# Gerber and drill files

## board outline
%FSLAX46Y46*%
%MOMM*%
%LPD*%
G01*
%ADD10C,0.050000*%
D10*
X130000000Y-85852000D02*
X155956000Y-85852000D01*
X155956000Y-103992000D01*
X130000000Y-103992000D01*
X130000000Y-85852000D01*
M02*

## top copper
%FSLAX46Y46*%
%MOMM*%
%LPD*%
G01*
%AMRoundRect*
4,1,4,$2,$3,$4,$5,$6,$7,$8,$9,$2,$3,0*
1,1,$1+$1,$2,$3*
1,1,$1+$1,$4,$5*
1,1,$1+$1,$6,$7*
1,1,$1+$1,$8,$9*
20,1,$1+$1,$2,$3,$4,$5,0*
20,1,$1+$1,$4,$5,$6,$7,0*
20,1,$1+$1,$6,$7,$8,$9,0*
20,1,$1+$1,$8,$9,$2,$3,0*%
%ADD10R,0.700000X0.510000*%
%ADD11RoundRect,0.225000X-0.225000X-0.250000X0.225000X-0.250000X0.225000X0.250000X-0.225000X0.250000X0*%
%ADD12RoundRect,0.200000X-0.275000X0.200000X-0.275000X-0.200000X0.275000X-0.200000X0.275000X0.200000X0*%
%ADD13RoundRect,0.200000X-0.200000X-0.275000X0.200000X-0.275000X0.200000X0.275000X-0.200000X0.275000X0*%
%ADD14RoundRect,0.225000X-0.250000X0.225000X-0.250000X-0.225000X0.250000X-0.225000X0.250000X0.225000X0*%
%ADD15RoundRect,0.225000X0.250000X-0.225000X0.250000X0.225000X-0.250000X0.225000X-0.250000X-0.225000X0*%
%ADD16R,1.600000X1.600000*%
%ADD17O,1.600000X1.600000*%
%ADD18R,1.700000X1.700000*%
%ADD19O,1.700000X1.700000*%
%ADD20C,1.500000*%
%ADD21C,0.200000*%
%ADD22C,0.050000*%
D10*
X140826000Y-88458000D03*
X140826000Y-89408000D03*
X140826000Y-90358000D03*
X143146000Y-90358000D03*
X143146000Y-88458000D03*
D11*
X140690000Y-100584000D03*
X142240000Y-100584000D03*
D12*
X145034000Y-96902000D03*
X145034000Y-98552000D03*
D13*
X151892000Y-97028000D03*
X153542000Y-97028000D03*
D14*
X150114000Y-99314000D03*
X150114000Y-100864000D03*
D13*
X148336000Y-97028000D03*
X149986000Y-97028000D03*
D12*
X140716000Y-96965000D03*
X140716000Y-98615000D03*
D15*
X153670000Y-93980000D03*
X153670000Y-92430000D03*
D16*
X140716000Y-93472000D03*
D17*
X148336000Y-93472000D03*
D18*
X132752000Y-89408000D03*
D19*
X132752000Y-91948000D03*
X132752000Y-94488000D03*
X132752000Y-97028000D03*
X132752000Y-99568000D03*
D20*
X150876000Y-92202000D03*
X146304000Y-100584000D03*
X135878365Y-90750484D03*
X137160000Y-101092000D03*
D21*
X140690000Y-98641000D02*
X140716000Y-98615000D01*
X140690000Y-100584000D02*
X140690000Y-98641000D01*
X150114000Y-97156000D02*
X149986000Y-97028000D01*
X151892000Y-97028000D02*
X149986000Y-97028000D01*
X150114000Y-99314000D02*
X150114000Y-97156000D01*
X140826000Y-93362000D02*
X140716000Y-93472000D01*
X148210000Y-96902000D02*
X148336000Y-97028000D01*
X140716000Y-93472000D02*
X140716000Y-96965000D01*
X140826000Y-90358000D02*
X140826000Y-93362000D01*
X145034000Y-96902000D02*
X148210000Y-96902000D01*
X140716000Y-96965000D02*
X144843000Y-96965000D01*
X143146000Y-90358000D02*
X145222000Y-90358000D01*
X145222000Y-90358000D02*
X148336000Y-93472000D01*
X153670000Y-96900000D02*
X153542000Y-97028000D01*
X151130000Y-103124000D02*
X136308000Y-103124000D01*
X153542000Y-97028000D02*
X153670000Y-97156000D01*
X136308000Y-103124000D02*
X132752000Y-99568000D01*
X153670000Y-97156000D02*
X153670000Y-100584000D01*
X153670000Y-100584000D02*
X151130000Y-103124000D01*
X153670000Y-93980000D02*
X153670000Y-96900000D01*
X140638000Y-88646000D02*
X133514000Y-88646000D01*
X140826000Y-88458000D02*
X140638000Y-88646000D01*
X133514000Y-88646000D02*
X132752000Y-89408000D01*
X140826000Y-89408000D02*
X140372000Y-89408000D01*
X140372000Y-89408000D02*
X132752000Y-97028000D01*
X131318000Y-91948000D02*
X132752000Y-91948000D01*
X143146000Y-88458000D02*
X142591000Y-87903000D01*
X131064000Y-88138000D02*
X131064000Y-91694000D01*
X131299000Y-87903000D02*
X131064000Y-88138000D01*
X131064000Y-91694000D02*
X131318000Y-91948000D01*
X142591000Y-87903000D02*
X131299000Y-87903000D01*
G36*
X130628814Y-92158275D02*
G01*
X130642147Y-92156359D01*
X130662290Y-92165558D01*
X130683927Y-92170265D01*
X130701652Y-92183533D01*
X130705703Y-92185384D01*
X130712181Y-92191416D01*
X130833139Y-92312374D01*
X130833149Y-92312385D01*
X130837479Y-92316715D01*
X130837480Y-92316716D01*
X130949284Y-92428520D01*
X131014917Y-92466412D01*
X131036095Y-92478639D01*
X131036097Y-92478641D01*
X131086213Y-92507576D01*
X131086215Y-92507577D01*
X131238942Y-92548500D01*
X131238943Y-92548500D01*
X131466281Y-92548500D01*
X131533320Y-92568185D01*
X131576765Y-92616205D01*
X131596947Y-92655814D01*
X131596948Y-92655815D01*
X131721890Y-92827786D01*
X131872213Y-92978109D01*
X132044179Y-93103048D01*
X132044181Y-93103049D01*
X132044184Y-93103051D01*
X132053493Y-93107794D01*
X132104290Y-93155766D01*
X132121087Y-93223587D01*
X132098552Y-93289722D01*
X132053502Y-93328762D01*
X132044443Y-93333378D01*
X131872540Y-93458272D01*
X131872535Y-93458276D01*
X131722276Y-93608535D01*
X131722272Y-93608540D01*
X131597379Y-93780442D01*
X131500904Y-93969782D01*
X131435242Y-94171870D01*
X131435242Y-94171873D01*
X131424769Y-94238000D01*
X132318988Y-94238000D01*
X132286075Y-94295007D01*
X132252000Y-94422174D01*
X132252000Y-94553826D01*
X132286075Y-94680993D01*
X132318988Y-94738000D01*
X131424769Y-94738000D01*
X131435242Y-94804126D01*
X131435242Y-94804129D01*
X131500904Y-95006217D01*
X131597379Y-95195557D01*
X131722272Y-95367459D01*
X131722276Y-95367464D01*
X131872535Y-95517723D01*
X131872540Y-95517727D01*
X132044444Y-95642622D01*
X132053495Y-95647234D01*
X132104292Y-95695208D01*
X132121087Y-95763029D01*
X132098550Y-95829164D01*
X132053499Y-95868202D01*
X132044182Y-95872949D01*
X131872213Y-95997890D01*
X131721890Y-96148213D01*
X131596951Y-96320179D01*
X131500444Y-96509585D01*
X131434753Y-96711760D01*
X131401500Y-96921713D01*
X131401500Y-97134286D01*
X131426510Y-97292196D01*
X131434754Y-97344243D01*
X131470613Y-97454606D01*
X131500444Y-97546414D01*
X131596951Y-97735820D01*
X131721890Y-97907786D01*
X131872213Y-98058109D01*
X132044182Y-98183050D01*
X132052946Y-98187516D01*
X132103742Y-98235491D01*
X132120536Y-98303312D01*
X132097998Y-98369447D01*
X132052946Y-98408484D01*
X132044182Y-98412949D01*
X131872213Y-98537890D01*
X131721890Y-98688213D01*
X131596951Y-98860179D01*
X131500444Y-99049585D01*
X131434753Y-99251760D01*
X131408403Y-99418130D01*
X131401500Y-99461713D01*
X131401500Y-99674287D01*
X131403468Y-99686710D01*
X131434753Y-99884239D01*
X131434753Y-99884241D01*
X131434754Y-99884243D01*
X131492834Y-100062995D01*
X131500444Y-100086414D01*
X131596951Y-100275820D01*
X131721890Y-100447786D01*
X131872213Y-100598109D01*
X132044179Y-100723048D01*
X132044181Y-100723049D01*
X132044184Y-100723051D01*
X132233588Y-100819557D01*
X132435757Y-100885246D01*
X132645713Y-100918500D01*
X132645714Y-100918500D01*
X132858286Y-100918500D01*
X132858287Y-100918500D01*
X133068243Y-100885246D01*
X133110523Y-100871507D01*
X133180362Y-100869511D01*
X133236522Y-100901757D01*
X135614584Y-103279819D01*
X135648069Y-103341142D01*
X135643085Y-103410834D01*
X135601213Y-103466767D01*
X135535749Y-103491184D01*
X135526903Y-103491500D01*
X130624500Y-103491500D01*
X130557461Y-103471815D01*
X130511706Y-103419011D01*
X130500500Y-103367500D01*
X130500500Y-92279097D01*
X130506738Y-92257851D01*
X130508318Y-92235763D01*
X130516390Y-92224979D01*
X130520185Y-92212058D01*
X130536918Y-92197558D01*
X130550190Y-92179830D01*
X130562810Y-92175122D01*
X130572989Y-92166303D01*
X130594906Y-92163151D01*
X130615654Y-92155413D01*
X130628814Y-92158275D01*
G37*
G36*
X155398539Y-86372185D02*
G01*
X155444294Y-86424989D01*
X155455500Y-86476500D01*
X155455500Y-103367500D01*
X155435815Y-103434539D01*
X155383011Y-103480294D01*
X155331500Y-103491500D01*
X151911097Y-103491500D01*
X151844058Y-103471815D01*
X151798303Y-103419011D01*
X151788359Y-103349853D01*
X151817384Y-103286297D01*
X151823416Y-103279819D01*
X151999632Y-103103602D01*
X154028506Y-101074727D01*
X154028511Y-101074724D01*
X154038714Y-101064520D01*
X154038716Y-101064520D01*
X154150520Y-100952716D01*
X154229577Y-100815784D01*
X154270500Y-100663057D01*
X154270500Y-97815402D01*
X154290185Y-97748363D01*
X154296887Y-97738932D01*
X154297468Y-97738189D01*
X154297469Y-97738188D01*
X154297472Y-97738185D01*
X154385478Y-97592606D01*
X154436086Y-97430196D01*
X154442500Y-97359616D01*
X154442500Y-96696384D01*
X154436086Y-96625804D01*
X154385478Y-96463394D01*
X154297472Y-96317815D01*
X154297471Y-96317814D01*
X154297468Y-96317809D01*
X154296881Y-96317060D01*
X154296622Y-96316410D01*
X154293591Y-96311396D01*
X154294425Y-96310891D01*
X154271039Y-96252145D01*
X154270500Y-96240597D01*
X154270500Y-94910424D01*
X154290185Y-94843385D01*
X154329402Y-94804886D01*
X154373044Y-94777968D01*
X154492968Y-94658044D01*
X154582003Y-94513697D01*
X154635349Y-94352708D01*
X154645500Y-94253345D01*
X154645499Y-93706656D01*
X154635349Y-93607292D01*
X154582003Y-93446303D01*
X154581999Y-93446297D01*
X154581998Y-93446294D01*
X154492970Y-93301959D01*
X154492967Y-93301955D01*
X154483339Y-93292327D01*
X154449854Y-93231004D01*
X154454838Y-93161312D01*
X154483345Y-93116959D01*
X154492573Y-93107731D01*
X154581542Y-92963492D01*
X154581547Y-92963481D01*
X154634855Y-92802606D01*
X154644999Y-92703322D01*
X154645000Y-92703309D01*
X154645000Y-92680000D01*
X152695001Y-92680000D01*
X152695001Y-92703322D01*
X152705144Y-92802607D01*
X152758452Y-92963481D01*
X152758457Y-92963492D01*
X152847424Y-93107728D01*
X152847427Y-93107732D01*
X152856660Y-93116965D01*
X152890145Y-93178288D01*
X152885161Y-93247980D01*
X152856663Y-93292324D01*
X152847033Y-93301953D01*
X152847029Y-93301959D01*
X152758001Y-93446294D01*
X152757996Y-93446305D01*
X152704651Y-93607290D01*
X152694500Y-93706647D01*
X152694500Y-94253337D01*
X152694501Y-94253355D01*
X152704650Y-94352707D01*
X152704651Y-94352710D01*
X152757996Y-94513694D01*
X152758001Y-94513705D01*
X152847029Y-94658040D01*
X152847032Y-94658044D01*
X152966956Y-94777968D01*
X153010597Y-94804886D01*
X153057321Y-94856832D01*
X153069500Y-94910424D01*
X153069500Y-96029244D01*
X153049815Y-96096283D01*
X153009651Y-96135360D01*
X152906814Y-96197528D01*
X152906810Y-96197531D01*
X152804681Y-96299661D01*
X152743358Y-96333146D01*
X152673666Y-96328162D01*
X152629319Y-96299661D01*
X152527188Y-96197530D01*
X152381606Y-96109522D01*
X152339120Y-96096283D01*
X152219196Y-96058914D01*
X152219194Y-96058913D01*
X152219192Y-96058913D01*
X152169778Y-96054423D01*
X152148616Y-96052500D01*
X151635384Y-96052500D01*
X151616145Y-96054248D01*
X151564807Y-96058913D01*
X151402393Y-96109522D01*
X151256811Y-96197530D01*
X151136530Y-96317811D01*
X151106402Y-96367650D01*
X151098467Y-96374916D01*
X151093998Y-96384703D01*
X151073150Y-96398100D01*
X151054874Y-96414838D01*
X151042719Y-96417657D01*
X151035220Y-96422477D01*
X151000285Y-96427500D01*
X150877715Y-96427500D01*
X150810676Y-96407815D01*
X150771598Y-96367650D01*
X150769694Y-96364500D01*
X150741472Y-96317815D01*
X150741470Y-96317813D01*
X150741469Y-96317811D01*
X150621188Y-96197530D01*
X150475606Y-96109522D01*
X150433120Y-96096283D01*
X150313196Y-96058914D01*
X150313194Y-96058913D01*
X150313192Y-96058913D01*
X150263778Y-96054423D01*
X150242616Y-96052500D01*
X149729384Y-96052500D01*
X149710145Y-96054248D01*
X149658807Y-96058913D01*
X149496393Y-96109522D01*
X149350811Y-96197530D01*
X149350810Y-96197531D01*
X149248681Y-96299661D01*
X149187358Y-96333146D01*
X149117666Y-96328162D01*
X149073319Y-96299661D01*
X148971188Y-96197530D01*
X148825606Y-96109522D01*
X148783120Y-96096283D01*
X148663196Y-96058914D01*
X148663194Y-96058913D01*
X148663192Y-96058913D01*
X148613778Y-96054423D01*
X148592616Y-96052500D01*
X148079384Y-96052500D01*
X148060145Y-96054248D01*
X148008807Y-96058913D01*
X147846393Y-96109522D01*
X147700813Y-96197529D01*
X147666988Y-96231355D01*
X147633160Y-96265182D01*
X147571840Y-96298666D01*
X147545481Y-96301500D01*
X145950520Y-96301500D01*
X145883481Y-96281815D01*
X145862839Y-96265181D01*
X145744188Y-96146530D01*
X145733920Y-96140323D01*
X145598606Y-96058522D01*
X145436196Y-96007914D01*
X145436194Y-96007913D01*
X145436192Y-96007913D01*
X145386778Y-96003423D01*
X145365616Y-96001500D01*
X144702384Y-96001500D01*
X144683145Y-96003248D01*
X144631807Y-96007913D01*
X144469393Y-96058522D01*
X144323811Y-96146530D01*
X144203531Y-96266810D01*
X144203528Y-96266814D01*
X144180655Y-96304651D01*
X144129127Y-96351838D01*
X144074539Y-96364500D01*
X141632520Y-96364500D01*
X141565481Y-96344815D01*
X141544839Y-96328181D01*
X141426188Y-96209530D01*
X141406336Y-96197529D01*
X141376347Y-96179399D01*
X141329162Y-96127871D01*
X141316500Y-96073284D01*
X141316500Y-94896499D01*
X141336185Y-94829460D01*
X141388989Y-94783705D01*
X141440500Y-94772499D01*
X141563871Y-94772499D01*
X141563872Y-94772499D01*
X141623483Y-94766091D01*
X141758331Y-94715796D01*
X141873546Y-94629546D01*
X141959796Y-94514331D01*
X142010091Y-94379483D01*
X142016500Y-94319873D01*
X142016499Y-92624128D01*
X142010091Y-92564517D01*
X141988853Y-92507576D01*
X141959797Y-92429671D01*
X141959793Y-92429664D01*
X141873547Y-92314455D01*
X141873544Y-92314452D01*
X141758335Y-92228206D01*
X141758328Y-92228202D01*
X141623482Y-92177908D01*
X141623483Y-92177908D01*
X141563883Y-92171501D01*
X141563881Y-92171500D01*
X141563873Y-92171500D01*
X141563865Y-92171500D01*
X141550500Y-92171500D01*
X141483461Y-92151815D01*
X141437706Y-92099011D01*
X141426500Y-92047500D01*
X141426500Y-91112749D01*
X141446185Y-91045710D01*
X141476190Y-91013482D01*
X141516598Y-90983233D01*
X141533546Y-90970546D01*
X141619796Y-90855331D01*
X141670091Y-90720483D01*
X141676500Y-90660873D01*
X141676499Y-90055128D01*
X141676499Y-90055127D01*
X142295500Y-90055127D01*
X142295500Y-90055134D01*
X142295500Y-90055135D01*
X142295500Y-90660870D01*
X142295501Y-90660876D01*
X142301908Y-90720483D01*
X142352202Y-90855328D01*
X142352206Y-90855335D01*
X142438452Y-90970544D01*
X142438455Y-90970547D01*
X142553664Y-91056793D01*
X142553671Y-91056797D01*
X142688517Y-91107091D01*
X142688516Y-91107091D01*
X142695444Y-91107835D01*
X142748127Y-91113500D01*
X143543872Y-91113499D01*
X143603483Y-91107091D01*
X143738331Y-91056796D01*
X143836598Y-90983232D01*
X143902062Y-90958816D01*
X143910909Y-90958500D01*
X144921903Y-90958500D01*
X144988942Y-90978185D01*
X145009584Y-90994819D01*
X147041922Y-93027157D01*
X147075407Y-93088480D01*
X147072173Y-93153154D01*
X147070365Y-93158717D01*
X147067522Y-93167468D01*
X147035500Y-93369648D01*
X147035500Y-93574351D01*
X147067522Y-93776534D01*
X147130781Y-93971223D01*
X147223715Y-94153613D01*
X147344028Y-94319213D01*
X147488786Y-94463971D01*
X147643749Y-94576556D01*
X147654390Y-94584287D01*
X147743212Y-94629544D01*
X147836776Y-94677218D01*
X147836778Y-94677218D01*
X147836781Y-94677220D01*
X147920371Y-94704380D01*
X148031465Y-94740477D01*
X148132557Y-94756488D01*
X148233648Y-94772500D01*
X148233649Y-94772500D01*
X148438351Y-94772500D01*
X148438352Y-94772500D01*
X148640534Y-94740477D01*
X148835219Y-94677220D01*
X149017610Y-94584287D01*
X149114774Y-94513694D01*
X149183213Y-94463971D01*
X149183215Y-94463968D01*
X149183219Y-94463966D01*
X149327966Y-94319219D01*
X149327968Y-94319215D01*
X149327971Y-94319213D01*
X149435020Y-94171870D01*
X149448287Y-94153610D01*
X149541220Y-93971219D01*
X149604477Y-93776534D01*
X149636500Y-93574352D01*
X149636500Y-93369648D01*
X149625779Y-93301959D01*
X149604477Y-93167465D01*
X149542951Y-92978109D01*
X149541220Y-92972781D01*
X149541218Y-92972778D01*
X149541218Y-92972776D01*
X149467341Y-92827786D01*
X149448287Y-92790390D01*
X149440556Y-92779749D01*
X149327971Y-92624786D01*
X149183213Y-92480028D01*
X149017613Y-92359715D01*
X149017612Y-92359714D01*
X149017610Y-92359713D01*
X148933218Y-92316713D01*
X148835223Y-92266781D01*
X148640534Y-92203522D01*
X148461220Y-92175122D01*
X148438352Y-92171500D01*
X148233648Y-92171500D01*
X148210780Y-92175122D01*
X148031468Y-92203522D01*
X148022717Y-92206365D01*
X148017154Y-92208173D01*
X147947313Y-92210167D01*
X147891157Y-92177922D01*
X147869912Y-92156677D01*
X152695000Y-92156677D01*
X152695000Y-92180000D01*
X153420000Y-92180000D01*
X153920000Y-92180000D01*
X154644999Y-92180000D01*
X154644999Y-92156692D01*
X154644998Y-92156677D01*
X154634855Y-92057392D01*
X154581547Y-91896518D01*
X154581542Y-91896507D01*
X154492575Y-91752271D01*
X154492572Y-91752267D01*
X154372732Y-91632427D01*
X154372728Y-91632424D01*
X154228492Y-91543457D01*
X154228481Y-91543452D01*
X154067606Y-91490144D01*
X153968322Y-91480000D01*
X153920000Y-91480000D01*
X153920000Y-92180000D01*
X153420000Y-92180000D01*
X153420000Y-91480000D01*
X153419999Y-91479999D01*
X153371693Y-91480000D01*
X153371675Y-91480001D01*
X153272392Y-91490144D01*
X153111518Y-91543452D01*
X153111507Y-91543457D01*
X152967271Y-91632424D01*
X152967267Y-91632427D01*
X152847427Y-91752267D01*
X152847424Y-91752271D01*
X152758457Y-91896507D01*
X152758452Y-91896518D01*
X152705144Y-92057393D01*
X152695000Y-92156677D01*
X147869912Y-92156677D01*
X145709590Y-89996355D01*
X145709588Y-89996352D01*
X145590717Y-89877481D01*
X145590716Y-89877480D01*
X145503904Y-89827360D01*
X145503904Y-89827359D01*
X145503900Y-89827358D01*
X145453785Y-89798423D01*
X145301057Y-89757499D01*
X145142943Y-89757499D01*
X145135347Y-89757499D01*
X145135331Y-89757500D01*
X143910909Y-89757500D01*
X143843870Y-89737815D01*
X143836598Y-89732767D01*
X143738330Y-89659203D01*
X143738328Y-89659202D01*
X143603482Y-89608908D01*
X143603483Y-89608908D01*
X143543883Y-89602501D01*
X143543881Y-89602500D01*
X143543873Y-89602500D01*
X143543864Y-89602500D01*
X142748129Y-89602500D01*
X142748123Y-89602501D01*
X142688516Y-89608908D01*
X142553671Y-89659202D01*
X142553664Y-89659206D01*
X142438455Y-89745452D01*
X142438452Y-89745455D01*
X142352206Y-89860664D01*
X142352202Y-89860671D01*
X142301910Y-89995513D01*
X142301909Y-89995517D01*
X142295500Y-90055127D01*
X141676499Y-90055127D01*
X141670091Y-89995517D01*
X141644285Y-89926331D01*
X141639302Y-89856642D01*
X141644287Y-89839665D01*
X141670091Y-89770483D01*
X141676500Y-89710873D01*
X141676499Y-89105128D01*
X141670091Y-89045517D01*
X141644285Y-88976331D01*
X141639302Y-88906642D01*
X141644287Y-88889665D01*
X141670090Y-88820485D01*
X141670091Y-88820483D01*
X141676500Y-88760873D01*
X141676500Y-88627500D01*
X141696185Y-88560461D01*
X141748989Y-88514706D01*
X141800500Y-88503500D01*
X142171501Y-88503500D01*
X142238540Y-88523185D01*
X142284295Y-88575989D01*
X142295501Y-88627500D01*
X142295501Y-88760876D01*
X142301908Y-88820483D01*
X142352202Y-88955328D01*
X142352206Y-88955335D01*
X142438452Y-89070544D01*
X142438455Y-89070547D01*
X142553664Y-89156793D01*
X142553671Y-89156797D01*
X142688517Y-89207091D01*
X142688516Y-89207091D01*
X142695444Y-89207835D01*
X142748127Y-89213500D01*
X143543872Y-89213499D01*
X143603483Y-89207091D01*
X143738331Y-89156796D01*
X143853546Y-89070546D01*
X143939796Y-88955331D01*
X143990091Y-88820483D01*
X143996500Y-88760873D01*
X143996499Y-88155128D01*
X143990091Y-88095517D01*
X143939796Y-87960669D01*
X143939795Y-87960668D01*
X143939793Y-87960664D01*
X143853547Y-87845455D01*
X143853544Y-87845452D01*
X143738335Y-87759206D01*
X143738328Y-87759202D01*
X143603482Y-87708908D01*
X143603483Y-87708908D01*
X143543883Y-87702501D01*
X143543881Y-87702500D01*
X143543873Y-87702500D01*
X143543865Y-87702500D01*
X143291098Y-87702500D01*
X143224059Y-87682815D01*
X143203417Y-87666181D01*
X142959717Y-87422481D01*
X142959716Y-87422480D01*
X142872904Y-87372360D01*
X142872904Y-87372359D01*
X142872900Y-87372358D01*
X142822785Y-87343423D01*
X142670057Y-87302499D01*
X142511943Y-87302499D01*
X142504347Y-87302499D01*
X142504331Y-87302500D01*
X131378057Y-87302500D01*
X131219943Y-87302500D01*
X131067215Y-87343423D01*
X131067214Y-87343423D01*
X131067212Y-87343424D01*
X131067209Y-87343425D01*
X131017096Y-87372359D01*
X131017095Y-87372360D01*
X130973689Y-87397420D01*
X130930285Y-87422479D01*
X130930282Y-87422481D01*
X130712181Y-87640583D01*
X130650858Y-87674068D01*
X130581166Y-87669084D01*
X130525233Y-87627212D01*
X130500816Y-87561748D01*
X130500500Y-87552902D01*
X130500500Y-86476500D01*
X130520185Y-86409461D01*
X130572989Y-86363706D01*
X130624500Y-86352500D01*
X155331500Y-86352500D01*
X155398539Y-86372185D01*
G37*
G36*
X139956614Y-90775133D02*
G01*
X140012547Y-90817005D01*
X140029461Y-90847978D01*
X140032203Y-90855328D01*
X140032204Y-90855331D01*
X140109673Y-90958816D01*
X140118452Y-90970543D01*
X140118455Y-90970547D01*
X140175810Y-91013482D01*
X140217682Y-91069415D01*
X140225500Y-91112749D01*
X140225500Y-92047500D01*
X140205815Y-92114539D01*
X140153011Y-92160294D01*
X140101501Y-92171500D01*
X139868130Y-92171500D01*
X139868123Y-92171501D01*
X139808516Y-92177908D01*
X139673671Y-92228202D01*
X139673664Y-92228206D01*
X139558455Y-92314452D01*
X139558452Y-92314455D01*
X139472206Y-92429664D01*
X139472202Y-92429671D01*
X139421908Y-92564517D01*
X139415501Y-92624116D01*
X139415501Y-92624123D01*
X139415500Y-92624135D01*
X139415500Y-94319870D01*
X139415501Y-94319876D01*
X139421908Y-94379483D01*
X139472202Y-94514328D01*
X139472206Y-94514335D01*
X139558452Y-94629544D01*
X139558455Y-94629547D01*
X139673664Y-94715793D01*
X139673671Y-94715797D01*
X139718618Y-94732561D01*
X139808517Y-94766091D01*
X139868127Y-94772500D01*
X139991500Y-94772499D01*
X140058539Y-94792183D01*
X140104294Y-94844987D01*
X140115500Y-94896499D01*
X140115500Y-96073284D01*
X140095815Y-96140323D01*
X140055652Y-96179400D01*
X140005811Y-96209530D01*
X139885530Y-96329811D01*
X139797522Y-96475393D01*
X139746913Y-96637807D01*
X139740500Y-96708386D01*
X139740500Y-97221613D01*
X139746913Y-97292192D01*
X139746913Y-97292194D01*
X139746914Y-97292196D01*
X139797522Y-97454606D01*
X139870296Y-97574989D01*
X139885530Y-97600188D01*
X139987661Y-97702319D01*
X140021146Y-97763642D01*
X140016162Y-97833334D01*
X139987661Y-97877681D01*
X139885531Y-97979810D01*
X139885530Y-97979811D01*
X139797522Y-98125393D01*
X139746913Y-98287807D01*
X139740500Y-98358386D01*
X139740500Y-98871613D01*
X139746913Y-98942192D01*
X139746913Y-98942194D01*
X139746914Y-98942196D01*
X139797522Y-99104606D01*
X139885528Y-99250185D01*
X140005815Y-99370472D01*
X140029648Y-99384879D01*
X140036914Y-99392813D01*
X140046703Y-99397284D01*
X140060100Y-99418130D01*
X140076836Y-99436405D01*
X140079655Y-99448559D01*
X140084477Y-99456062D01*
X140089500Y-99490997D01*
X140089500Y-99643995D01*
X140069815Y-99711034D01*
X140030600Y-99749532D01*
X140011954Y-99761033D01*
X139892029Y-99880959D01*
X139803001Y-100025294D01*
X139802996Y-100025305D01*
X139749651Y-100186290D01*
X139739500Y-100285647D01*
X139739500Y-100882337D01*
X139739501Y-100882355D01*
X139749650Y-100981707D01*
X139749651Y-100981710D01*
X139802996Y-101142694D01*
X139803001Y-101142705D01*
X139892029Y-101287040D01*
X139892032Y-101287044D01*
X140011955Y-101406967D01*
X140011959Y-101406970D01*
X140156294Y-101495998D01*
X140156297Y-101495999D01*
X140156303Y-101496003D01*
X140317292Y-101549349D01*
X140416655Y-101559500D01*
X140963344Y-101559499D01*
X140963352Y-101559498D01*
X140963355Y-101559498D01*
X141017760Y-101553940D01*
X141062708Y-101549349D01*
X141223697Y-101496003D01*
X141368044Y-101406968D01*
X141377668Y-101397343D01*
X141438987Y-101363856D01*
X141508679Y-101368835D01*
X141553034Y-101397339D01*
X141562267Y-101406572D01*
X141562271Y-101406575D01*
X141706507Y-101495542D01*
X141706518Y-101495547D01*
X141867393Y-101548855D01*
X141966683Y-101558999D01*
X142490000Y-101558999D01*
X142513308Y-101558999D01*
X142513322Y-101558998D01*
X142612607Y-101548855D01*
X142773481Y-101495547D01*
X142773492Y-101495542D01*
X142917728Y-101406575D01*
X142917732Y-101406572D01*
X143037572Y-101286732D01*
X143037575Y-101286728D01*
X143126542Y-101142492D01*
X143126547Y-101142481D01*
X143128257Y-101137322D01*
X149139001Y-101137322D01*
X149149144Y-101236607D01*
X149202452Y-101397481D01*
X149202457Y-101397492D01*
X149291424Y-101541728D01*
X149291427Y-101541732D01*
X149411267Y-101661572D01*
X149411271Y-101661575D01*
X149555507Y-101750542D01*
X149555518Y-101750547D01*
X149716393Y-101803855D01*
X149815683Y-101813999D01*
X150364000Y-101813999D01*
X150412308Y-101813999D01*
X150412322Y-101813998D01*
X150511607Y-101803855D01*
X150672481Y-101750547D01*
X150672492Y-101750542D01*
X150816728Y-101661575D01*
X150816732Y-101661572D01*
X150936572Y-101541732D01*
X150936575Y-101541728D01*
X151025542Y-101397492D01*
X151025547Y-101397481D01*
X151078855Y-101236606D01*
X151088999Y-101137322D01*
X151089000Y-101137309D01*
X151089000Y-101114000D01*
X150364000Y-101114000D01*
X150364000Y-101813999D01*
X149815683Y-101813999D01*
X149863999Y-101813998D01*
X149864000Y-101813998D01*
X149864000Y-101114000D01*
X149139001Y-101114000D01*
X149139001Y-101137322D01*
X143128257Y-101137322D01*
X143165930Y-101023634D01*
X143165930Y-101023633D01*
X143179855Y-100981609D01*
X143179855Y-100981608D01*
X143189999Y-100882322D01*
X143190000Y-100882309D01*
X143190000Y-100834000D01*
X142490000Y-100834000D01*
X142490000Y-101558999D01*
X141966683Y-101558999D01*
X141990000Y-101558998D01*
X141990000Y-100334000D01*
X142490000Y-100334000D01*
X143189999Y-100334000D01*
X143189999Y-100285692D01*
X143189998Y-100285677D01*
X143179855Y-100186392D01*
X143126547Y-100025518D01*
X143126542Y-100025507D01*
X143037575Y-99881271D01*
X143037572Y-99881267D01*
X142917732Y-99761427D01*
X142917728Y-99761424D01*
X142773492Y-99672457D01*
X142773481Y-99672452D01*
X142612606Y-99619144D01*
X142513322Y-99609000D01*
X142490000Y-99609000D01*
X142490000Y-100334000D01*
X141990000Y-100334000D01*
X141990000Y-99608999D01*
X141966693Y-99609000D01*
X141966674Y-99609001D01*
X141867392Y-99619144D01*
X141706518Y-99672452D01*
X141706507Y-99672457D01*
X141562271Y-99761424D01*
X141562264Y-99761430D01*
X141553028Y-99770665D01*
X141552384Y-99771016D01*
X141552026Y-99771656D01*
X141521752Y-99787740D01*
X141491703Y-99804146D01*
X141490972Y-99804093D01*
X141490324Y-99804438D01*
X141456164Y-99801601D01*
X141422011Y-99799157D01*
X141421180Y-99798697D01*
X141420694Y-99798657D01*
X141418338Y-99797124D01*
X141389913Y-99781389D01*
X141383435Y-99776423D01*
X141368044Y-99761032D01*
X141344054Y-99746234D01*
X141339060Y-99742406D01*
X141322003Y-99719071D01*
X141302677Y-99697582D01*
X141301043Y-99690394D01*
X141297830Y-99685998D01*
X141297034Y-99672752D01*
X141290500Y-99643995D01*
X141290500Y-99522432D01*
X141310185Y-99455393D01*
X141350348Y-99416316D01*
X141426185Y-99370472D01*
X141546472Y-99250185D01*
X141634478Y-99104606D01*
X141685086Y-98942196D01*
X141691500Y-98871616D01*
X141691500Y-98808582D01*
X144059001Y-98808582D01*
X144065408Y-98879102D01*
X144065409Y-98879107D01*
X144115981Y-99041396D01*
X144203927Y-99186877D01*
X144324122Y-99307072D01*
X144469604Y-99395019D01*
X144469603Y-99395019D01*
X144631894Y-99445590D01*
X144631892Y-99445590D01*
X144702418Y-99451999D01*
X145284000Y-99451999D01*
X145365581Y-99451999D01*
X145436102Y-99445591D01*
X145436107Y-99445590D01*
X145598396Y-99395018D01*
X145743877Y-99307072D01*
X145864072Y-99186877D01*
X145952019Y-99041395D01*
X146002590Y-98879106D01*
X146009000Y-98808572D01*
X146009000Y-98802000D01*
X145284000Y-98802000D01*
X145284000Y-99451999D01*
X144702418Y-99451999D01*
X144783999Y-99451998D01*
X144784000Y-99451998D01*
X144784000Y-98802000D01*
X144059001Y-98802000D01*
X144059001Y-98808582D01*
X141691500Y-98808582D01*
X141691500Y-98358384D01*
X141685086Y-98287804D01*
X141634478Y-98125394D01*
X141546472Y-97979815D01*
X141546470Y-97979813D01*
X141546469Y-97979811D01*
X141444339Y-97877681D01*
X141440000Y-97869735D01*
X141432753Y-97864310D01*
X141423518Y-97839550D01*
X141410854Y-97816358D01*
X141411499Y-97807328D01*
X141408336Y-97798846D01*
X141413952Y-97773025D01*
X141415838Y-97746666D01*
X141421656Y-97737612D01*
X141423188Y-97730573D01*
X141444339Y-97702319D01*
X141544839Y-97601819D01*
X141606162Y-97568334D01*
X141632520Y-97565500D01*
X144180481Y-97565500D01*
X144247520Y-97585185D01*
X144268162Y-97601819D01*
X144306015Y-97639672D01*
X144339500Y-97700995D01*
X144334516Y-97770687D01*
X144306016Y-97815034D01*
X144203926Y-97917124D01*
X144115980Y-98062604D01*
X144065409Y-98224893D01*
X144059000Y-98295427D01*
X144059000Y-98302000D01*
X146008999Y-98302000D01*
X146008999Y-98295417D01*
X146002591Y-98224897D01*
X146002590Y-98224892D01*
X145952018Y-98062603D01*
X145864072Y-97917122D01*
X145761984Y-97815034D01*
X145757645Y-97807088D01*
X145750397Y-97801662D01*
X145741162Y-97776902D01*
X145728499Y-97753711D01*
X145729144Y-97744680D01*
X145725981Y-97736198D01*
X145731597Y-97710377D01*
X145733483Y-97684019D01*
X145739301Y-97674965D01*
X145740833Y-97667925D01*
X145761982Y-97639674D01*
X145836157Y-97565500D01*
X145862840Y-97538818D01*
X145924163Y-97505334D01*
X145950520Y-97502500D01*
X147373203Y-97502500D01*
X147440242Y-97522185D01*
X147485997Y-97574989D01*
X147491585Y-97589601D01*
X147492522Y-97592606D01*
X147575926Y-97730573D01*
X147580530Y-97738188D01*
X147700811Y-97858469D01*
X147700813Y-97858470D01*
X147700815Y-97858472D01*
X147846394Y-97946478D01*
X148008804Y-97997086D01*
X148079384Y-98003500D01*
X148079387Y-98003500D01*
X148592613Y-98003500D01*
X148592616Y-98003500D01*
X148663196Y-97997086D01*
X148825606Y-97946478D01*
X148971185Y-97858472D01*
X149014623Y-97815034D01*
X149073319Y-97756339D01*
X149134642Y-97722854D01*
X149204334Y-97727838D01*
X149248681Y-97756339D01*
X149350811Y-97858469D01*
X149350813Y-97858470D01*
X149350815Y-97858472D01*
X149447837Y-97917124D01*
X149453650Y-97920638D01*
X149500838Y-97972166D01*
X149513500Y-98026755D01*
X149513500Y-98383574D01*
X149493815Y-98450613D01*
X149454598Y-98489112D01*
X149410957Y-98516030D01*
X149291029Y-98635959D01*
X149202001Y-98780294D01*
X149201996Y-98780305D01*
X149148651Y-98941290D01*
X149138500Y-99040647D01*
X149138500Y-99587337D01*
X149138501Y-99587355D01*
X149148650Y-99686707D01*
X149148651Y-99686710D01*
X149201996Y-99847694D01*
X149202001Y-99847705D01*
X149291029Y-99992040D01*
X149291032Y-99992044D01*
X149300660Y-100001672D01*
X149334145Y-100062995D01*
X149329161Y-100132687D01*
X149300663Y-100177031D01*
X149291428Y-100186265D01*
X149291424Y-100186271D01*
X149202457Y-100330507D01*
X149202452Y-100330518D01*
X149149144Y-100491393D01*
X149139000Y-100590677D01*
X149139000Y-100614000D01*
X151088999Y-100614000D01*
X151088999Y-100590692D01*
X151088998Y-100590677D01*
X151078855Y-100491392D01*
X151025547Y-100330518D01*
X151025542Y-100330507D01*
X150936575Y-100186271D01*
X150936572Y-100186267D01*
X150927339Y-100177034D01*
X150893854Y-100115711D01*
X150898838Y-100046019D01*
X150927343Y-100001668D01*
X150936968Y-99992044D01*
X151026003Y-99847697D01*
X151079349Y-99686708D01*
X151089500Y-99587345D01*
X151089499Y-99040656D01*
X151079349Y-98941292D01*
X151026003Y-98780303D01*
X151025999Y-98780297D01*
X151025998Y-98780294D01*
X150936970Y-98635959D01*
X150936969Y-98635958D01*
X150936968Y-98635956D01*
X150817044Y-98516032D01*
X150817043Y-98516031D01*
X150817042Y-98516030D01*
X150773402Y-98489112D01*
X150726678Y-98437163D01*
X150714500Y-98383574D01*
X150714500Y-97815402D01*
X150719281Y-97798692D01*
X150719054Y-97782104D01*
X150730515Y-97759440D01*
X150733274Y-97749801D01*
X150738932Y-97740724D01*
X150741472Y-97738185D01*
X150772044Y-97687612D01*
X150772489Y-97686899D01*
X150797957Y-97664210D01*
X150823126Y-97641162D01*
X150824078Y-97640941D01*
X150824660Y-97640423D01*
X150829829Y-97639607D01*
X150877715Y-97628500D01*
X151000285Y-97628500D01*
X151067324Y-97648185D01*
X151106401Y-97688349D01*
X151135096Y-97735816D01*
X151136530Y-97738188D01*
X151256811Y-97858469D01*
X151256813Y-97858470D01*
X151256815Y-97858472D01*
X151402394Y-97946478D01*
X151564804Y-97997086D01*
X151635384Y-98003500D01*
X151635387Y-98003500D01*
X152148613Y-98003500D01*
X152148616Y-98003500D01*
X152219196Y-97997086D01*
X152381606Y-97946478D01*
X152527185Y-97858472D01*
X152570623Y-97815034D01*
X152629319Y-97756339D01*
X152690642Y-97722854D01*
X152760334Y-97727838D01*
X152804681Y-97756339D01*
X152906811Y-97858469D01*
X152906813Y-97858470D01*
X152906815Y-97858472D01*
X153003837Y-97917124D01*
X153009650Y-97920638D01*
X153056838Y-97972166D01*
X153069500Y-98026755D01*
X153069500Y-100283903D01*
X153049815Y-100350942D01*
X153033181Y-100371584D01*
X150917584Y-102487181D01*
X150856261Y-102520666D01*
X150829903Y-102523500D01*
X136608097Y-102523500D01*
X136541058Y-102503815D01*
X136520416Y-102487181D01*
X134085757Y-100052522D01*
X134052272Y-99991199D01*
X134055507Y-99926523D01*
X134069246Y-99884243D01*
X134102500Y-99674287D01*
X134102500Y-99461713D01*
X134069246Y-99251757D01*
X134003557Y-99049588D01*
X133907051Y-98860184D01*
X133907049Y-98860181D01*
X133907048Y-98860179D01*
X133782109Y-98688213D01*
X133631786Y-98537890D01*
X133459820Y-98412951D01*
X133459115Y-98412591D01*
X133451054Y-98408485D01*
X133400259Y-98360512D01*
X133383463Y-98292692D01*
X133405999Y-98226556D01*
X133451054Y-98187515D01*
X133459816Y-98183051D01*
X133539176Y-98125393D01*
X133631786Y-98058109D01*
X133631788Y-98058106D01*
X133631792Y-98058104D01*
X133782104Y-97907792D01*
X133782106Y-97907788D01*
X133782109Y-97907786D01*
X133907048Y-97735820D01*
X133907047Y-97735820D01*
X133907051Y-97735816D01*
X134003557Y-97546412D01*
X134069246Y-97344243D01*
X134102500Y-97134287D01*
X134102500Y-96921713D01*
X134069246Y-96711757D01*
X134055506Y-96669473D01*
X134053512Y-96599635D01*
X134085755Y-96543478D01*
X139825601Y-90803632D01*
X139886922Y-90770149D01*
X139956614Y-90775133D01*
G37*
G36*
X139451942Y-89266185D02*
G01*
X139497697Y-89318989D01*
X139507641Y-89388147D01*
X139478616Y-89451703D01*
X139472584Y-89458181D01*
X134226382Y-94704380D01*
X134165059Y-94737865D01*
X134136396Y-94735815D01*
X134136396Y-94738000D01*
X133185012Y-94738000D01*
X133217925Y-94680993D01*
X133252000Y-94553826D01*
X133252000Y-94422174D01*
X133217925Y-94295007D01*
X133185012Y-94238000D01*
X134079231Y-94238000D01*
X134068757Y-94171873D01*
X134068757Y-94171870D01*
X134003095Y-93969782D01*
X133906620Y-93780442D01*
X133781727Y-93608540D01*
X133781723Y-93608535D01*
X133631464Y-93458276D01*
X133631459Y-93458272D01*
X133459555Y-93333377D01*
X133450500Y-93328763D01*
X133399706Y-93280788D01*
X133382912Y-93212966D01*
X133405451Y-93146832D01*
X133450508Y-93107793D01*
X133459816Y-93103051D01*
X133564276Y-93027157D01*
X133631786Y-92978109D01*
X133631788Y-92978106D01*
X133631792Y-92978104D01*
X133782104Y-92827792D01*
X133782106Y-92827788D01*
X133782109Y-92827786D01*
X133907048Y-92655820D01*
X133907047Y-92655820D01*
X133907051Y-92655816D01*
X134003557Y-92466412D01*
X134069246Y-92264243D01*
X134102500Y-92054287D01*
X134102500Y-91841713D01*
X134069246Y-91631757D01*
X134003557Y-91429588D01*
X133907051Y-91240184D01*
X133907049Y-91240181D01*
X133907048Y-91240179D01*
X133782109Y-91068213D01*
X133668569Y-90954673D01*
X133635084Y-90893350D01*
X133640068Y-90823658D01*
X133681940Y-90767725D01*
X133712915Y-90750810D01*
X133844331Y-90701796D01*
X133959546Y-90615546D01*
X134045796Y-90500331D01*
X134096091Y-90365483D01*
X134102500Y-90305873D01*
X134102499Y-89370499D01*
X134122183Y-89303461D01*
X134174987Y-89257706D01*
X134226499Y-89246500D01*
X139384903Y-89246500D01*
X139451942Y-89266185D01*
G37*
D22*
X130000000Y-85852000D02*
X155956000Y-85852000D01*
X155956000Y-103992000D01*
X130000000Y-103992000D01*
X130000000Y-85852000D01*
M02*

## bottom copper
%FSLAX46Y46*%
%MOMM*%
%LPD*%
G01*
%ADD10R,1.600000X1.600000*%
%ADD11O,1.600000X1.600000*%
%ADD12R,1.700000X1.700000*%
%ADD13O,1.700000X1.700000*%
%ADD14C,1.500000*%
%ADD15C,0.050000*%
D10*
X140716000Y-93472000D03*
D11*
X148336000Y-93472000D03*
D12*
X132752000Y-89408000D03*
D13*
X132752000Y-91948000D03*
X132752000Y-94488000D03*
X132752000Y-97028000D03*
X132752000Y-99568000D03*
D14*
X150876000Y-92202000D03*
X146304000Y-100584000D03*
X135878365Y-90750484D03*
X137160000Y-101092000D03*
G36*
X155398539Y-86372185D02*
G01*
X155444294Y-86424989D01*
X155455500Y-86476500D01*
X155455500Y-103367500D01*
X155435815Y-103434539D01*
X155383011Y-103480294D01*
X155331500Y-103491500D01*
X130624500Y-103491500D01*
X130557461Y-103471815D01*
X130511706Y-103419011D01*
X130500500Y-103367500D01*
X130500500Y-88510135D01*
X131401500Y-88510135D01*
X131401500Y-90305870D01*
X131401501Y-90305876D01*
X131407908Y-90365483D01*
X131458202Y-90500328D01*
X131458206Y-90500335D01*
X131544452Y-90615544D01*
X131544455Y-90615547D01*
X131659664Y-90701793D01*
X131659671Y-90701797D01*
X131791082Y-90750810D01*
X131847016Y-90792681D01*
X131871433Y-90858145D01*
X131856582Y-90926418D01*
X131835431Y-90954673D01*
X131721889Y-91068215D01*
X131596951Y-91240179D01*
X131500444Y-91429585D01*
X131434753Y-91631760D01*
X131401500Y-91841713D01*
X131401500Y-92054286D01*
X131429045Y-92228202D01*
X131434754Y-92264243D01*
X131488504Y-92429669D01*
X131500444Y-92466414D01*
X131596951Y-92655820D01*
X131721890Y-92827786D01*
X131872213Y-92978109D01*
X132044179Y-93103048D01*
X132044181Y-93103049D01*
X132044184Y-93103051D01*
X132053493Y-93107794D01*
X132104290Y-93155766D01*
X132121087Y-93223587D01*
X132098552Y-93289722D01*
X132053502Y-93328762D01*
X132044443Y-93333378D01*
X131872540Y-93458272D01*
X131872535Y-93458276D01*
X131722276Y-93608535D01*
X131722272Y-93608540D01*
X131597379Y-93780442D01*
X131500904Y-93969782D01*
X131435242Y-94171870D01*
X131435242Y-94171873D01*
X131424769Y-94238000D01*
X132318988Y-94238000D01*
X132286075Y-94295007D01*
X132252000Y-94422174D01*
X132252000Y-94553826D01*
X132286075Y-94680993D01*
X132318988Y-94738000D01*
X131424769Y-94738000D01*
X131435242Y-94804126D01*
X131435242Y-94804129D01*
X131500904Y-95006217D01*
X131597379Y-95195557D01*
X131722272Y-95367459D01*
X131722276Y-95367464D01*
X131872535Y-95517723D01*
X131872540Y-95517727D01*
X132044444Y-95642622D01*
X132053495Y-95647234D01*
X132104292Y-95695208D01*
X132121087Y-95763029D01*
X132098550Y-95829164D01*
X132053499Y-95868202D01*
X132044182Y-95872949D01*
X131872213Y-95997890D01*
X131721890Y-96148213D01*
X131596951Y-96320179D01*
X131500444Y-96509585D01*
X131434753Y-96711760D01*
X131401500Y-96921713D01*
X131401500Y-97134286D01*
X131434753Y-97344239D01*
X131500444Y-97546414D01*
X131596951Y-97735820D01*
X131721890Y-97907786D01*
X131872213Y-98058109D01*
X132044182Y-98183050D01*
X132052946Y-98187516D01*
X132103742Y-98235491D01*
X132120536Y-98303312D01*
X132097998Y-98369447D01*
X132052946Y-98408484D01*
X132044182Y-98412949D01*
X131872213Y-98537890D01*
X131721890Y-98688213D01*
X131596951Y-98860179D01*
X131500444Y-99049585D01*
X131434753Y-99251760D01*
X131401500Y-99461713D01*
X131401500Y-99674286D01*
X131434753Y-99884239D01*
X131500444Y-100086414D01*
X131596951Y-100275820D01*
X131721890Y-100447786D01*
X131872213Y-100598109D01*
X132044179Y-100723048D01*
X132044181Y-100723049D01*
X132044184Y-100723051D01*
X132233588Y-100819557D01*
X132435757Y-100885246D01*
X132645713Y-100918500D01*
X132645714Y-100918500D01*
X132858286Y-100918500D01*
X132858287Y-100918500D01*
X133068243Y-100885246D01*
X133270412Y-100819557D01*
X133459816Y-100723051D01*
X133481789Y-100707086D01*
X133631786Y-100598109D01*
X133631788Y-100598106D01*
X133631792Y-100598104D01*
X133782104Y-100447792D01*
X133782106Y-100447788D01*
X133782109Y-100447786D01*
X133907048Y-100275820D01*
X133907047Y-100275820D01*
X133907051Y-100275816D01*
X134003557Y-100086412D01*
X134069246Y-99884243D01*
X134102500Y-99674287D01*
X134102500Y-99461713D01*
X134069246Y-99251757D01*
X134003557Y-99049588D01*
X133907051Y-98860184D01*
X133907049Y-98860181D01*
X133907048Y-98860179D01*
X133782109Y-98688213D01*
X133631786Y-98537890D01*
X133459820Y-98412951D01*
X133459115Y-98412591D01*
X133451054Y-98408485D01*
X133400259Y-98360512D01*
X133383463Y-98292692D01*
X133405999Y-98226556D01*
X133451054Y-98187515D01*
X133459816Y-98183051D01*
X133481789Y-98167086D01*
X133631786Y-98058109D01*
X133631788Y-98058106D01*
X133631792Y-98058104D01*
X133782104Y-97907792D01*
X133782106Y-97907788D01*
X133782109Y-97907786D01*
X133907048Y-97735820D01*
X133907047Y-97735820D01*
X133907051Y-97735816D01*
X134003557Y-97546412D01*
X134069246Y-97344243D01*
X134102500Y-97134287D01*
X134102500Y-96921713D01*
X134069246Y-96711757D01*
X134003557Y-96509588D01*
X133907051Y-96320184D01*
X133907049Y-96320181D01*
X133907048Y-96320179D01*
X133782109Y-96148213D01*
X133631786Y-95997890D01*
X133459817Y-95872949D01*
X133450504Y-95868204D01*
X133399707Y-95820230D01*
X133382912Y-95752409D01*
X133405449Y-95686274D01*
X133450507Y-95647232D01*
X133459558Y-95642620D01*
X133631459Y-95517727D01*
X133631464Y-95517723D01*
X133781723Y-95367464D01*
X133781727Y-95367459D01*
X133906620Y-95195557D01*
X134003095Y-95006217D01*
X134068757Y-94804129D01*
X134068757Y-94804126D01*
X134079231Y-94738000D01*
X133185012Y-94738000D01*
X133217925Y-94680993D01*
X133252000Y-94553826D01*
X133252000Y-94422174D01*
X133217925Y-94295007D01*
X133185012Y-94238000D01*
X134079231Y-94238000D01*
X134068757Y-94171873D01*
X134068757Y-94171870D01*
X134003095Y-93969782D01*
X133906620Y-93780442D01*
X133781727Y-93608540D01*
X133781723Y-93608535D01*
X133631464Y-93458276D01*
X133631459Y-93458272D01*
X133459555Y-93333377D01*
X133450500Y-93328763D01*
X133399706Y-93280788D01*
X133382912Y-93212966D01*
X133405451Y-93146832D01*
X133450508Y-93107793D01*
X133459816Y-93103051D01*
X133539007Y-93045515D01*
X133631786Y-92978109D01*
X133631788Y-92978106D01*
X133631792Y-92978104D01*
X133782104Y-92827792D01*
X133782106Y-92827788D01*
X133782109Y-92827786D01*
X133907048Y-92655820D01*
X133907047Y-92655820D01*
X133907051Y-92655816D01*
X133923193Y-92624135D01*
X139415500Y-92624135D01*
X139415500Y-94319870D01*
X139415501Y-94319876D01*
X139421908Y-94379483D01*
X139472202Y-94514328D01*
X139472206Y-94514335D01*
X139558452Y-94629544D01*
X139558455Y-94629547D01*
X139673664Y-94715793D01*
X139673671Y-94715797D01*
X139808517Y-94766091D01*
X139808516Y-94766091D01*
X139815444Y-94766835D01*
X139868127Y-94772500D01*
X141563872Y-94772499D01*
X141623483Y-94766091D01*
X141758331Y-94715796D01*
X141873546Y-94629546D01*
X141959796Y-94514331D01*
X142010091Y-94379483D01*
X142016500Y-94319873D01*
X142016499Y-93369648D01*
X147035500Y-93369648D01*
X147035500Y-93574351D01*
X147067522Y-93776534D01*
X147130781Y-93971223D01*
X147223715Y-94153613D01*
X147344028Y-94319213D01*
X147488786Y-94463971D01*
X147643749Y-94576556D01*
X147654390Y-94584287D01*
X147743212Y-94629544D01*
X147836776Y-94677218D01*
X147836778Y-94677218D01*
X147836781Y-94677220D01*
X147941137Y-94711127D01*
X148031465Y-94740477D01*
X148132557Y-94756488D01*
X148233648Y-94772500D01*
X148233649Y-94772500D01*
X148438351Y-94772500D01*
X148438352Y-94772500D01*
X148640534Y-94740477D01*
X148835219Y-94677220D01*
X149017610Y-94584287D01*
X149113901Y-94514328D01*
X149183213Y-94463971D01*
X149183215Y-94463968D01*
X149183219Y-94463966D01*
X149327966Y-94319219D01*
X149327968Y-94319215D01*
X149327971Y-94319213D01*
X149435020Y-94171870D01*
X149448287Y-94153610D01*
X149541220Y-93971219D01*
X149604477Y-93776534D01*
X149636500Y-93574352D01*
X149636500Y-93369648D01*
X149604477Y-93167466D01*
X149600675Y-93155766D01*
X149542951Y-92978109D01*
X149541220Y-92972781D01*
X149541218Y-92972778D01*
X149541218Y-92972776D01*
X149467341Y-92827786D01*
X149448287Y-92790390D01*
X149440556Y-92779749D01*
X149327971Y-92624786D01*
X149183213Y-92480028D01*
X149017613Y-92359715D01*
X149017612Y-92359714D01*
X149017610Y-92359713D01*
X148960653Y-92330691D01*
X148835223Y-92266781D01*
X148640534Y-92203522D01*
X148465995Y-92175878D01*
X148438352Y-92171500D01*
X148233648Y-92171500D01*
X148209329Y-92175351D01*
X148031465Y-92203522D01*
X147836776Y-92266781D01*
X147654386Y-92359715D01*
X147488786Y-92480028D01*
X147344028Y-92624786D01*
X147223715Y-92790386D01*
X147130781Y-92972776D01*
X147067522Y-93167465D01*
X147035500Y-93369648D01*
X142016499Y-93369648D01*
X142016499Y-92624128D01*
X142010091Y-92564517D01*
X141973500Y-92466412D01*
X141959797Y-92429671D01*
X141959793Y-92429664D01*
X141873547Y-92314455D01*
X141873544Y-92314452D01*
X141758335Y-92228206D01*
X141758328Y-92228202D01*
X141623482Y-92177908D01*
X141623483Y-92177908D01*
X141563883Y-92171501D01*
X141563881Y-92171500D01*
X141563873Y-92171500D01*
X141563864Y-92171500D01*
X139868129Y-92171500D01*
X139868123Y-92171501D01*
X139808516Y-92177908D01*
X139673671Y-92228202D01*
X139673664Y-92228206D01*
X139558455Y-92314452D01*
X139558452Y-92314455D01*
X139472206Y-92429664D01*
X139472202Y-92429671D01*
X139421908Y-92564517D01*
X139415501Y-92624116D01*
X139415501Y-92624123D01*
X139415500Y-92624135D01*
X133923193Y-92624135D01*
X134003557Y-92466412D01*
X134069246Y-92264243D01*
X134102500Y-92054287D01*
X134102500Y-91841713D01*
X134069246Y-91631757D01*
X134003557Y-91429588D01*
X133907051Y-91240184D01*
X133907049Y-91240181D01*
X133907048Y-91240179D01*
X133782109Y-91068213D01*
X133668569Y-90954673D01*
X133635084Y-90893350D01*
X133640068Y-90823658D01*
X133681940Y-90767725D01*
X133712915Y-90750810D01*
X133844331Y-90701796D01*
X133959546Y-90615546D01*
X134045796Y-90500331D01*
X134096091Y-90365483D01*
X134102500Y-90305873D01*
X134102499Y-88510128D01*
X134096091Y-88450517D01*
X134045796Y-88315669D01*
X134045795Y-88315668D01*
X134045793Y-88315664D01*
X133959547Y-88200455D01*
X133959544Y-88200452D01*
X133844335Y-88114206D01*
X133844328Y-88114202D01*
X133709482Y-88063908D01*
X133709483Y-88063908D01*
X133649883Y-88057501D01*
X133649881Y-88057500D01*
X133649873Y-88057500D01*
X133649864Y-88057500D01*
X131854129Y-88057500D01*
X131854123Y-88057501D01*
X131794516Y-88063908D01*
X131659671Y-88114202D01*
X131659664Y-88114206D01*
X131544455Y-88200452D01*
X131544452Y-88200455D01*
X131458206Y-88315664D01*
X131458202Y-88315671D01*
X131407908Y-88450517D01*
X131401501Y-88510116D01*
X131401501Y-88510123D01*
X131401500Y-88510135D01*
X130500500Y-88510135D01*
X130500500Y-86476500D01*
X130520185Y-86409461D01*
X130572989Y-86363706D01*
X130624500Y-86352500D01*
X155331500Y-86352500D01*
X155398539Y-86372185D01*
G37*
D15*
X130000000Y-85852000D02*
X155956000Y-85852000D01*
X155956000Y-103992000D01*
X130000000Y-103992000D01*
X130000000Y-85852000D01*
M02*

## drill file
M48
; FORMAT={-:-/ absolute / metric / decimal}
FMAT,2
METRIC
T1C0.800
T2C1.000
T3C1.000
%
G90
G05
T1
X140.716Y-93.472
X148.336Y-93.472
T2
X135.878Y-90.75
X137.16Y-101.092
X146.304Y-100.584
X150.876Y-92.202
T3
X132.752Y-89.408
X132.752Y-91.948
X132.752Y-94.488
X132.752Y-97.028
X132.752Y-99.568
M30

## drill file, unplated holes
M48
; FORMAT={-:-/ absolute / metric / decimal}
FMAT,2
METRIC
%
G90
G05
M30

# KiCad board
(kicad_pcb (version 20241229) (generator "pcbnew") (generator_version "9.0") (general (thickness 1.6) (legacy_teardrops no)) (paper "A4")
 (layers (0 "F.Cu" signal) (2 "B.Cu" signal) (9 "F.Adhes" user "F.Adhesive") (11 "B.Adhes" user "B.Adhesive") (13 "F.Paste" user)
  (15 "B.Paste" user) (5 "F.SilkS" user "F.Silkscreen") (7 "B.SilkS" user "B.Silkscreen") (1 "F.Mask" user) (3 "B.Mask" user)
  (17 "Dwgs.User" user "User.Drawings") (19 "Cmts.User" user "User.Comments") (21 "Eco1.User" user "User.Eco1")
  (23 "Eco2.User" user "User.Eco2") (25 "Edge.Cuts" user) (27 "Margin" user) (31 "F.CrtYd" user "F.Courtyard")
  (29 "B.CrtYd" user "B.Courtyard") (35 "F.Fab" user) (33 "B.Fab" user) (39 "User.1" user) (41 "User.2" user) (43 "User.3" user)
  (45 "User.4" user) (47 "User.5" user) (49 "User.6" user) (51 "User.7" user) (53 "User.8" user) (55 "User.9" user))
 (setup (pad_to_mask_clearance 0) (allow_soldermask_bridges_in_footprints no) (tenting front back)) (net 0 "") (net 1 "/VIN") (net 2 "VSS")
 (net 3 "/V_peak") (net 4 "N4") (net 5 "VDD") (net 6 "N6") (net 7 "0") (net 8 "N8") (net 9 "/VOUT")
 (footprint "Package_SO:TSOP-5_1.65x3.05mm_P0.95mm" (layer "F.Cu") (at 141.986 89.408)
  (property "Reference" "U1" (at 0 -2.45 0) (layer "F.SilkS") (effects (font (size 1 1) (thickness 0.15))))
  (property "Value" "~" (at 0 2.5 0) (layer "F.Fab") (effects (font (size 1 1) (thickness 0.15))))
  (pad "1" smd rect (at -1.16 -0.95) (size 0.7 0.51) (layers "F.Cu" "F.Mask" "F.Paste") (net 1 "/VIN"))
  (pad "2" smd rect (at -1.16 0) (size 0.7 0.51) (layers "F.Cu" "F.Mask" "F.Paste") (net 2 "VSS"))
  (pad "3" smd rect (at -1.16 0.95) (size 0.7 0.51) (layers "F.Cu" "F.Mask" "F.Paste") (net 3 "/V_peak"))
  (pad "4" smd rect (at 1.16 0.95) (size 0.7 0.51) (layers "F.Cu" "F.Mask" "F.Paste") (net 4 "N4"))
  (pad "5" smd rect (at 1.16 -0.95) (size 0.7 0.51) (layers "F.Cu" "F.Mask" "F.Paste") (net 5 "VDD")))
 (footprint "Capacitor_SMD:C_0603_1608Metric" (layer "F.Cu") (at 141.465 100.584)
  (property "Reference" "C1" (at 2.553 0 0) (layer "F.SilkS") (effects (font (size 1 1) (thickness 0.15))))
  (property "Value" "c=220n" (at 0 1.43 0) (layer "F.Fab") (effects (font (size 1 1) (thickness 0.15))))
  (pad "1" smd roundrect (at -0.775 0) (size 0.9 0.95) (layers "F.Cu" "F.Mask" "F.Paste") (roundrect_rratio 0.25) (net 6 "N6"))
  (pad "2" smd roundrect (at 0.775 0) (size 0.9 0.95) (layers "F.Cu" "F.Mask" "F.Paste") (roundrect_rratio 0.25) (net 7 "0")))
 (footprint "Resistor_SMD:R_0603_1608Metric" (layer "F.Cu") (at 145.034 97.727 -90)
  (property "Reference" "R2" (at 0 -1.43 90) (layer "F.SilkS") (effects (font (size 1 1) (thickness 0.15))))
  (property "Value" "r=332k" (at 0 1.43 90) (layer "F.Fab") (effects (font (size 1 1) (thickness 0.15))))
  (pad "1" smd roundrect (at -0.825 0 270) (size 0.8 0.95) (layers "F.Cu" "F.Mask" "F.Paste") (roundrect_rratio 0.25) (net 3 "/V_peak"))
  (pad "2" smd roundrect (at 0.825 0 270) (size 0.8 0.95) (layers "F.Cu" "F.Mask" "F.Paste") (roundrect_rratio 0.25) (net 7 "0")))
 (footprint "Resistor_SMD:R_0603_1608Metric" (layer "F.Cu") (at 152.717 97.028)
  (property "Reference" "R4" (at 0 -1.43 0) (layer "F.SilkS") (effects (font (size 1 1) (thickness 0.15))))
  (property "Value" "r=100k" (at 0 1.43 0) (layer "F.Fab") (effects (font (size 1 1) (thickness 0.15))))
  (pad "1" smd roundrect (at -0.825 0) (size 0.8 0.95) (layers "F.Cu" "F.Mask" "F.Paste") (roundrect_rratio 0.25) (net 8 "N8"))
  (pad "2" smd roundrect (at 0.825 0) (size 0.8 0.95) (layers "F.Cu" "F.Mask" "F.Paste") (roundrect_rratio 0.25) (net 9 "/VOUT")))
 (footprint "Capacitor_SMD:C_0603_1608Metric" (layer "F.Cu") (at 150.114 100.089 -90)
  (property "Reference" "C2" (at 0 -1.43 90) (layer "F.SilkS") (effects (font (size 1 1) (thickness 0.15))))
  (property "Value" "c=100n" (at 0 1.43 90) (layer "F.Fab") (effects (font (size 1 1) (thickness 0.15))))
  (pad "1" smd roundrect (at -0.775 0 270) (size 0.9 0.95) (layers "F.Cu" "F.Mask" "F.Paste") (roundrect_rratio 0.25) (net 8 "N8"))
  (pad "2" smd roundrect (at 0.775 0 270) (size 0.9 0.95) (layers "F.Cu" "F.Mask" "F.Paste") (roundrect_rratio 0.25) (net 7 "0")))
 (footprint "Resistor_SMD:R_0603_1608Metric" (layer "F.Cu") (at 149.161 97.028)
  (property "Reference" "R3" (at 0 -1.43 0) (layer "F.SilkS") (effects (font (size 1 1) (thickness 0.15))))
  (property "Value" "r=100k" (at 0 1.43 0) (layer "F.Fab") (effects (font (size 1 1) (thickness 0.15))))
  (pad "1" smd roundrect (at -0.825 0) (size 0.8 0.95) (layers "F.Cu" "F.Mask" "F.Paste") (roundrect_rratio 0.25) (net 3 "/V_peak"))
  (pad "2" smd roundrect (at 0.825 0) (size 0.8 0.95) (layers "F.Cu" "F.Mask" "F.Paste") (roundrect_rratio 0.25) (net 8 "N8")))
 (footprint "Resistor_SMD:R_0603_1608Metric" (layer "F.Cu") (at 140.716 97.79 -90)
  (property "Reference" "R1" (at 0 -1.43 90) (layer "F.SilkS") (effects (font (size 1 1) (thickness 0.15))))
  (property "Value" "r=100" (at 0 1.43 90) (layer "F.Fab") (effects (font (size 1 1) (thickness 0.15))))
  (pad "1" smd roundrect (at -0.825 0 270) (size 0.8 0.95) (layers "F.Cu" "F.Mask" "F.Paste") (roundrect_rratio 0.25) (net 3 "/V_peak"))
  (pad "2" smd roundrect (at 0.825 0 270) (size 0.8 0.95) (layers "F.Cu" "F.Mask" "F.Paste") (roundrect_rratio 0.25) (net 6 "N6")))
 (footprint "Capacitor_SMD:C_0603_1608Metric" (layer "F.Cu") (at 153.67 93.205 90)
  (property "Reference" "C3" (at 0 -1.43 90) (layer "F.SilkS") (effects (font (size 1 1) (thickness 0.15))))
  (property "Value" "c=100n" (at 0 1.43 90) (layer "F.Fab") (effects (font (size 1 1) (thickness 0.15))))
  (pad "1" smd roundrect (at -0.775 0 90) (size 0.9 0.95) (layers "F.Cu" "F.Mask" "F.Paste") (roundrect_rratio 0.25) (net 9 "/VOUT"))
  (pad "2" smd roundrect (at 0.775 0 90) (size 0.9 0.95) (layers "F.Cu" "F.Mask" "F.Paste") (roundrect_rratio 0.25) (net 7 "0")))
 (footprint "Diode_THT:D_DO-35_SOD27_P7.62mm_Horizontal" (layer "F.Cu") (at 140.716 93.472)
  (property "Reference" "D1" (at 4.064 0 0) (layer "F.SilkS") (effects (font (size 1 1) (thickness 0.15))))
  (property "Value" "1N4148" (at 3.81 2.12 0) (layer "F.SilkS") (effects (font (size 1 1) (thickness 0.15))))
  (pad "1" thru_hole rect (at 0 0) (size 1.6 1.6) (drill 0.8) (layers "*.Cu" "*.Mask") (remove_unused_layers no) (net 3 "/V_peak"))
  (pad "2" thru_hole oval (at 7.62 0) (size 1.6 1.6) (drill 0.8) (layers "*.Cu" "*.Mask") (remove_unused_layers no) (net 4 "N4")))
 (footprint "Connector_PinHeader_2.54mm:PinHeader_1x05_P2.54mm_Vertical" (layer "B.Cu") (at 132.752 89.408 180)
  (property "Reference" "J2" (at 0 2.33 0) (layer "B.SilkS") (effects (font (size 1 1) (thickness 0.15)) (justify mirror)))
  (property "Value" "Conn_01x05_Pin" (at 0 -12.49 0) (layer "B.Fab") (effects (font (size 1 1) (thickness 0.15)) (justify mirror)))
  (pad "1" thru_hole rect (at 0 0 180) (size 1.7 1.7) (drill 1) (layers "*.Cu" "*.Mask") (remove_unused_layers no) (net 1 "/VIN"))
  (pad "2" thru_hole oval (at 0 -2.54 180) (size 1.7 1.7) (drill 1) (layers "*.Cu" "*.Mask") (remove_unused_layers no) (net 5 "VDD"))
  (pad "3" thru_hole oval (at 0 -5.08 180) (size 1.7 1.7) (drill 1) (layers "*.Cu" "*.Mask") (remove_unused_layers no) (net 7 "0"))
  (pad "4" thru_hole oval (at 0 -7.62 180) (size 1.7 1.7) (drill 1) (layers "*.Cu" "*.Mask") (remove_unused_layers no) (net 2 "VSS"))
  (pad "5" thru_hole oval (at 0 -10.16 180) (size 1.7 1.7) (drill 1) (layers "*.Cu" "*.Mask") (remove_unused_layers no) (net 9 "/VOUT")))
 (gr_rect (start 130 85.852) (end 155.956 103.992) (stroke (width 0.05) (type default)) (fill no) (layer "Edge.Cuts"))
 (via (at 150.876 92.202) (size 1.5) (drill 1) (layers "F.Cu" "B.Cu") (free yes) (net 7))
 (via (at 146.304 100.584) (size 1.5) (drill 1) (layers "F.Cu" "B.Cu") (free yes) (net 7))
 (via (at 135.878365 90.750484) (size 1.5) (drill 1) (layers "F.Cu" "B.Cu") (free yes) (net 7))
 (via (at 137.16 101.092) (size 1.5) (drill 1) (layers "F.Cu" "B.Cu") (free yes) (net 7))
 (segment (start 140.69 98.641) (end 140.716 98.615) (width 0.2) (layer "F.Cu") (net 6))
 (segment (start 140.69 100.584) (end 140.69 98.641) (width 0.2) (layer "F.Cu") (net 6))
 (segment (start 150.114 97.156) (end 149.986 97.028) (width 0.2) (layer "F.Cu") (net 8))
 (segment (start 151.892 97.028) (end 149.986 97.028) (width 0.2) (layer "F.Cu") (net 8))
 (segment (start 150.114 99.314) (end 150.114 97.156) (width 0.2) (layer "F.Cu") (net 8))
 (segment (start 140.826 93.362) (end 140.716 93.472) (width 0.2) (layer "F.Cu") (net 3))
 (segment (start 148.21 96.902) (end 148.336 97.028) (width 0.2) (layer "F.Cu") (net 3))
 (segment (start 140.716 93.472) (end 140.716 96.965) (width 0.2) (layer "F.Cu") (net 3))
 (segment (start 140.826 90.358) (end 140.826 93.362) (width 0.2) (layer "F.Cu") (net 3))
 (segment (start 145.034 96.902) (end 148.21 96.902) (width 0.2) (layer "F.Cu") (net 3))
 (segment (start 140.716 96.965) (end 144.843 96.965) (width 0.2) (layer "F.Cu") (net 3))
 (segment (start 143.146 90.358) (end 145.222 90.358) (width 0.2) (layer "F.Cu") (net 4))
 (segment (start 145.222 90.358) (end 148.336 93.472) (width 0.2) (layer "F.Cu") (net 4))
 (segment (start 153.67 96.9) (end 153.542 97.028) (width 0.2) (layer "F.Cu") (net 9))
 (segment (start 151.13 103.124) (end 136.308 103.124) (width 0.2) (layer "F.Cu") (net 9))
 (segment (start 153.542 97.028) (end 153.67 97.156) (width 0.2) (layer "F.Cu") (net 9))
 (segment (start 136.308 103.124) (end 132.752 99.568) (width 0.2) (layer "F.Cu") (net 9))
 (segment (start 153.67 97.156) (end 153.67 100.584) (width 0.2) (layer "F.Cu") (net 9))
 (segment (start 153.67 100.584) (end 151.13 103.124) (width 0.2) (layer "F.Cu") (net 9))
 (segment (start 153.67 93.98) (end 153.67 96.9) (width 0.2) (layer "F.Cu") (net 9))
 (segment (start 140.638 88.646) (end 133.514 88.646) (width 0.2) (layer "F.Cu") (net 1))
 (segment (start 140.826 88.458) (end 140.638 88.646) (width 0.2) (layer "F.Cu") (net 1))
 (segment (start 133.514 88.646) (end 132.752 89.408) (width 0.2) (layer "F.Cu") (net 1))
 (segment (start 140.826 89.408) (end 140.372 89.408) (width 0.2) (layer "F.Cu") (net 2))
 (segment (start 140.372 89.408) (end 132.752 97.028) (width 0.2) (layer "F.Cu") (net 2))
 (segment (start 131.318 91.948) (end 132.752 91.948) (width 0.2) (layer "F.Cu") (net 5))
 (segment (start 143.146 88.458) (end 142.591 87.903) (width 0.2) (layer "F.Cu") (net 5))
 (segment (start 131.064 88.138) (end 131.064 91.694) (width 0.2) (layer "F.Cu") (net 5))
 (segment (start 131.299 87.903) (end 131.064 88.138) (width 0.2) (layer "F.Cu") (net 5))
 (segment (start 131.064 91.694) (end 131.318 91.948) (width 0.2) (layer "F.Cu") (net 5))
 (segment (start 142.591 87.903) (end 131.299 87.903) (width 0.2) (layer "F.Cu") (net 5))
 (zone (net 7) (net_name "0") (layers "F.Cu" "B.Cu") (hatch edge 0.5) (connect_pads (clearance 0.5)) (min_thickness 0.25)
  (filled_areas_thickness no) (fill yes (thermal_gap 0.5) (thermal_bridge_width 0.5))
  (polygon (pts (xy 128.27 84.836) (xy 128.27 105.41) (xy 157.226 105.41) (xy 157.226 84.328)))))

